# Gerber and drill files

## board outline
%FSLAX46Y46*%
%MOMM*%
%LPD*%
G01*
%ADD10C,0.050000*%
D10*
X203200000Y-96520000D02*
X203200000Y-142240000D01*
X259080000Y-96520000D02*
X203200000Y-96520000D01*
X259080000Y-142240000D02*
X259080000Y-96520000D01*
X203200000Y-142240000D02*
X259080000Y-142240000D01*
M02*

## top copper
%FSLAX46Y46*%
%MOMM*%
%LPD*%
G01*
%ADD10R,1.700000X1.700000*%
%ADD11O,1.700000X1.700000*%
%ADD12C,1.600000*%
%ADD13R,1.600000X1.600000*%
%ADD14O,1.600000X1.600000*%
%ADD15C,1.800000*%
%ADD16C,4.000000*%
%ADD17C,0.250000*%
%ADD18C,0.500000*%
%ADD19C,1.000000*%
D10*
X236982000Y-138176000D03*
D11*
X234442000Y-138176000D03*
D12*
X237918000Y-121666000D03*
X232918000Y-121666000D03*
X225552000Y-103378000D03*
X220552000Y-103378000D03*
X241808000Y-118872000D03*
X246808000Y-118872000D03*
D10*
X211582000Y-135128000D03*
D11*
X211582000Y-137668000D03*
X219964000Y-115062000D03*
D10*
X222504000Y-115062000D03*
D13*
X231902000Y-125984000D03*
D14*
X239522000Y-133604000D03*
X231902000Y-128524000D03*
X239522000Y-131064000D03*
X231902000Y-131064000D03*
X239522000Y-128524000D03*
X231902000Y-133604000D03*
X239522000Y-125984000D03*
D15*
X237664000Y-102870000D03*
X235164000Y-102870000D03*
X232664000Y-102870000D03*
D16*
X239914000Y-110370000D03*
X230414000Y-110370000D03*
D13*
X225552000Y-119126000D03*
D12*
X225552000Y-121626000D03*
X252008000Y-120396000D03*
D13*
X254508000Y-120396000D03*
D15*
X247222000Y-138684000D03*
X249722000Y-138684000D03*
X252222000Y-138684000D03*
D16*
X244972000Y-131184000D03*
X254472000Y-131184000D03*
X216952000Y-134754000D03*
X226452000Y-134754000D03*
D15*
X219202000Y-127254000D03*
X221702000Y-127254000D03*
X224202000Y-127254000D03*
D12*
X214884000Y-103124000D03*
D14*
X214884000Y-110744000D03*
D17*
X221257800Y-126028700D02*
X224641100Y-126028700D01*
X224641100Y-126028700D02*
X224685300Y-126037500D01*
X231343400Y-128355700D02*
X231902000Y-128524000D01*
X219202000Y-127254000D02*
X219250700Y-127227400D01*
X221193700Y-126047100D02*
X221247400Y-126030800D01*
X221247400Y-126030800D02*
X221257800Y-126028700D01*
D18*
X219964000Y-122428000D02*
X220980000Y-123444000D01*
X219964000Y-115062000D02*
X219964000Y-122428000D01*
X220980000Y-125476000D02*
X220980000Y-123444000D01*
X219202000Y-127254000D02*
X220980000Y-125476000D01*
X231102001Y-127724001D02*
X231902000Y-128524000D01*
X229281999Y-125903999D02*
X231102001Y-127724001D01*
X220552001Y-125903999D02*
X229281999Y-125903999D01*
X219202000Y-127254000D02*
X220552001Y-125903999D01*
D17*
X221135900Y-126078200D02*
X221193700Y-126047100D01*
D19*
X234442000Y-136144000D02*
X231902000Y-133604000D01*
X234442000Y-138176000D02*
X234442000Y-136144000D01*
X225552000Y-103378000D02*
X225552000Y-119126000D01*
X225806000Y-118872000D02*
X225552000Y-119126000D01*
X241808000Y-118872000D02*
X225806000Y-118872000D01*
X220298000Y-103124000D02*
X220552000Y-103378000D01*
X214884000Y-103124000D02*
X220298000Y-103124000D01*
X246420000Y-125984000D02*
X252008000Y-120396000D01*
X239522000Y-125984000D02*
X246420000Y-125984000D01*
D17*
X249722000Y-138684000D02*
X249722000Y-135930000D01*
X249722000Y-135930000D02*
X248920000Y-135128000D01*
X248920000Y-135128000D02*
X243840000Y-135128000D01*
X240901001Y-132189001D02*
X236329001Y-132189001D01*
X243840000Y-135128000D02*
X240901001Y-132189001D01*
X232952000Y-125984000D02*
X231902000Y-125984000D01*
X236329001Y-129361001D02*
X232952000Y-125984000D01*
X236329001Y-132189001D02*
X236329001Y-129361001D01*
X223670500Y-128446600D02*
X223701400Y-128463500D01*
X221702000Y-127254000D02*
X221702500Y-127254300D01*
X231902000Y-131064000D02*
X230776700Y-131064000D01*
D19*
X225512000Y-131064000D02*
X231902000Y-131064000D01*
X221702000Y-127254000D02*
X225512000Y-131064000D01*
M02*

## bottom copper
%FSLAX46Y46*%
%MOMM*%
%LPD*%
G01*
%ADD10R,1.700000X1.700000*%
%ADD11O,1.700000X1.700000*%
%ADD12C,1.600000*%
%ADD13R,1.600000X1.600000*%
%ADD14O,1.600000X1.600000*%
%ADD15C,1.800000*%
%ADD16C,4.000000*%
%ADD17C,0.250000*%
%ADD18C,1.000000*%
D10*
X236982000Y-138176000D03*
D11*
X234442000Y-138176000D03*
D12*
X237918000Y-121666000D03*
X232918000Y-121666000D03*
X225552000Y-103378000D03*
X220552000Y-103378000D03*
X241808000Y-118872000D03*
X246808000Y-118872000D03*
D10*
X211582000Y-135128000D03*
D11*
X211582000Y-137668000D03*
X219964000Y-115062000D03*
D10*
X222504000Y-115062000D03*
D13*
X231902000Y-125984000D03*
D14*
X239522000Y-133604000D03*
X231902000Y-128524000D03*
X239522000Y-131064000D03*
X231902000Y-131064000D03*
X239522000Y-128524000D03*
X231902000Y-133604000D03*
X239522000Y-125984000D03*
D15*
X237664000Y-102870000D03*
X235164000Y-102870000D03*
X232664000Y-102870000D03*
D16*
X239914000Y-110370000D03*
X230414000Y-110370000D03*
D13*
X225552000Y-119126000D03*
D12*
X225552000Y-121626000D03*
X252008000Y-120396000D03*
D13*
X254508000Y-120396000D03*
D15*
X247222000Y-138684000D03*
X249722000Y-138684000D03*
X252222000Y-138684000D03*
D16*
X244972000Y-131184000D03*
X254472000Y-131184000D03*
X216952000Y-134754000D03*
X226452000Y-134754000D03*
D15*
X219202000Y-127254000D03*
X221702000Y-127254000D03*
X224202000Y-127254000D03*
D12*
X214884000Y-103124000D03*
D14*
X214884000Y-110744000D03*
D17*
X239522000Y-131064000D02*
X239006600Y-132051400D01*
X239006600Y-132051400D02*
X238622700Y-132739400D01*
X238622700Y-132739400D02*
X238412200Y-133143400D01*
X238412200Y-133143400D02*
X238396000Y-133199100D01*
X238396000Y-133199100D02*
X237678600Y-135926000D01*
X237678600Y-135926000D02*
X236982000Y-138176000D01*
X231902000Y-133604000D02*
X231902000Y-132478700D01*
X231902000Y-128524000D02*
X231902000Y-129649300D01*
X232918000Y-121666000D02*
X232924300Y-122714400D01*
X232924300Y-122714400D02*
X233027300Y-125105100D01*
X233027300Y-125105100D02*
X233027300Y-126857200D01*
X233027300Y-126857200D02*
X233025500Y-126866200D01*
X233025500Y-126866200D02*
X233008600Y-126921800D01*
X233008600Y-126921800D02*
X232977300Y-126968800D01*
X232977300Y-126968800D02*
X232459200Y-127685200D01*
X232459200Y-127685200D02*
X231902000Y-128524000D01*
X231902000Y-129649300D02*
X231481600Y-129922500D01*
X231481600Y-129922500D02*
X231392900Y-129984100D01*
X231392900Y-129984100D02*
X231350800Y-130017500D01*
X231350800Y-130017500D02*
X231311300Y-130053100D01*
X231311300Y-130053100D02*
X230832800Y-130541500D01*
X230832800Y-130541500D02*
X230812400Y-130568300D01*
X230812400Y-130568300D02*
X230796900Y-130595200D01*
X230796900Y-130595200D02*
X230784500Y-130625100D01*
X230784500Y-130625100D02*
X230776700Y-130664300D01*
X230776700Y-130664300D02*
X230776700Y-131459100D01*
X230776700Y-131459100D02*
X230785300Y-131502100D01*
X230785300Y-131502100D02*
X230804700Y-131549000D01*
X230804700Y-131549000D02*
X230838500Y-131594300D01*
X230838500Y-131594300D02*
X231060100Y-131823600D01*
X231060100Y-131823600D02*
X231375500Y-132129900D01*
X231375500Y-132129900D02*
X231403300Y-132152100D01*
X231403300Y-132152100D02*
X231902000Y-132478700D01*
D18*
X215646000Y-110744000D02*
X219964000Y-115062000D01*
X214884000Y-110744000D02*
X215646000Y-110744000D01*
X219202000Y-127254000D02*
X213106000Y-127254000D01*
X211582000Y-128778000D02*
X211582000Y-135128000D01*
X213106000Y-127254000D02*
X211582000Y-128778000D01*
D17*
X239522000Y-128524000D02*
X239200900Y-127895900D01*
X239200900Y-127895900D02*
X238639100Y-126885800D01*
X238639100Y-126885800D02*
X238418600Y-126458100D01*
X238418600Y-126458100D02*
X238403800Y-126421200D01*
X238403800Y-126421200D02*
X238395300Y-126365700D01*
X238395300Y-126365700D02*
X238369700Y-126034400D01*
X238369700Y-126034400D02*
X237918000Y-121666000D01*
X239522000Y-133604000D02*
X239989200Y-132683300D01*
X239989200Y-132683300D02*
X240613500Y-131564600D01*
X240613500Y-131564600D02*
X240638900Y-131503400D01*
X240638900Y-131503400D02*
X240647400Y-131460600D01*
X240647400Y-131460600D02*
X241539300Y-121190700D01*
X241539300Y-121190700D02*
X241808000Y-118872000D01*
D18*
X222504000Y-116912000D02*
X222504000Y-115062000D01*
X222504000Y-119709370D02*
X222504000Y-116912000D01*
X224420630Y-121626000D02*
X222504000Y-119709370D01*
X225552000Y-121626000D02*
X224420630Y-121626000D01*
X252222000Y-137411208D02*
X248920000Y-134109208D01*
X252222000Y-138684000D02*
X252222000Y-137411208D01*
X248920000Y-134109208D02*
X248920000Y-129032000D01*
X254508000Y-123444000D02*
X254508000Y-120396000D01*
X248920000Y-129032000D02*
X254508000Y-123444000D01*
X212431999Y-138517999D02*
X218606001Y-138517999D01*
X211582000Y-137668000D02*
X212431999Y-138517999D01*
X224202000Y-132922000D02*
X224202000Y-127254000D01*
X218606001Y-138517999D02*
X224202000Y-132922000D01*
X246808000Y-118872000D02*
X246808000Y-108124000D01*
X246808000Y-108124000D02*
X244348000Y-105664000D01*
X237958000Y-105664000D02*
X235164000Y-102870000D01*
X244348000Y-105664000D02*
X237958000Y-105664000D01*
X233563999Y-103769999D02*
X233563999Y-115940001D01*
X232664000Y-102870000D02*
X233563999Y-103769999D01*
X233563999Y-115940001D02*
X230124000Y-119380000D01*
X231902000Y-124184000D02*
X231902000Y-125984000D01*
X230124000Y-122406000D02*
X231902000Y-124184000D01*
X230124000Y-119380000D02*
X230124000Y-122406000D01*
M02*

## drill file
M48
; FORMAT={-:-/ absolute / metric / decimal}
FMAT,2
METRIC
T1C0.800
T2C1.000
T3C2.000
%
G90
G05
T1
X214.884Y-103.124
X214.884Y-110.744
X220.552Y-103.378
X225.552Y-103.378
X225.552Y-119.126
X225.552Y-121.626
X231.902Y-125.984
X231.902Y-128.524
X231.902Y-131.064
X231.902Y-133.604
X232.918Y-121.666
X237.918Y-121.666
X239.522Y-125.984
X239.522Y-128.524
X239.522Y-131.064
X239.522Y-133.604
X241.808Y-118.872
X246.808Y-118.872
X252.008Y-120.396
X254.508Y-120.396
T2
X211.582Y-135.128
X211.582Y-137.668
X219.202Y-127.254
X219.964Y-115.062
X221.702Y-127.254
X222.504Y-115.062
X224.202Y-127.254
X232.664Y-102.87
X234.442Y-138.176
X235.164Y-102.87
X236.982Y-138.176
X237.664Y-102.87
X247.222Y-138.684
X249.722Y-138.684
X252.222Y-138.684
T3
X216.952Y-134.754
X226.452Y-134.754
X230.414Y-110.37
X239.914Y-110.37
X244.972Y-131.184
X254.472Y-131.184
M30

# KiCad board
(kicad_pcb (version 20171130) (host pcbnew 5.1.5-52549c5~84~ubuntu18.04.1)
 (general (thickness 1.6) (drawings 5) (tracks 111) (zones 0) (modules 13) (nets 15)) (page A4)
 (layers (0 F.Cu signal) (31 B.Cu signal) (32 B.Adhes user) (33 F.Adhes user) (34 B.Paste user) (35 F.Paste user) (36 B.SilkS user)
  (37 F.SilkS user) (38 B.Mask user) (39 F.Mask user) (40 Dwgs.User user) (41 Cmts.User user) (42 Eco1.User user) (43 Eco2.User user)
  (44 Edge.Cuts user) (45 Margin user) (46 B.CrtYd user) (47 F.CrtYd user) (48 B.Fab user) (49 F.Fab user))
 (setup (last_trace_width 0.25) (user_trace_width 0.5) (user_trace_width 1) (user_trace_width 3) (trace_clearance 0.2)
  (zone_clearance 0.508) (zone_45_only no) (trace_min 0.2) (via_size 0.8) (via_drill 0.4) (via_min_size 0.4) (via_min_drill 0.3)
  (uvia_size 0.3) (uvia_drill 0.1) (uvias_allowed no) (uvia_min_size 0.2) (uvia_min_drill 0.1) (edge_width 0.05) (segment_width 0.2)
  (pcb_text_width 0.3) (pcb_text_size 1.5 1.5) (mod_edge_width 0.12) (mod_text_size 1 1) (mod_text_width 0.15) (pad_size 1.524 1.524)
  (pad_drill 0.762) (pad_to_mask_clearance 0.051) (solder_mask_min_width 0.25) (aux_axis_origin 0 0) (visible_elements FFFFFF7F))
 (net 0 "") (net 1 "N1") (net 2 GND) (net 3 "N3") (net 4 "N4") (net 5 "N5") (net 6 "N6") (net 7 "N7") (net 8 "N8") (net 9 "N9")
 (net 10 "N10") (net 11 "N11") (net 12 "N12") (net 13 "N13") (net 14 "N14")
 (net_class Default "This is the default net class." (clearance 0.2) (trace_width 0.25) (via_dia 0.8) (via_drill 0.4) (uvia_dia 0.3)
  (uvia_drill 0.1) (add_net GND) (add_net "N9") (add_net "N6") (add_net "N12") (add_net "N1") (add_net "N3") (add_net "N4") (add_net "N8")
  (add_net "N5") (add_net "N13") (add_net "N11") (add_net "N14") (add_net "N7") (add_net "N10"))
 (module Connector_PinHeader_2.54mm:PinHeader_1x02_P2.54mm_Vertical (layer F.Cu) (at 236.982 138.176 270)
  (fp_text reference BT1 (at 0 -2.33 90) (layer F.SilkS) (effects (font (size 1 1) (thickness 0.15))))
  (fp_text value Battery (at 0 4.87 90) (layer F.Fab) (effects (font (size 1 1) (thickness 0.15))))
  (pad 1 thru_hole rect (at 0 0 270) (size 1.7 1.7) (drill 1) (layers *.Cu *.Mask) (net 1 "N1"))
  (pad 2 thru_hole oval (at 0 2.54 270) (size 1.7 1.7) (drill 1) (layers *.Cu *.Mask) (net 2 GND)))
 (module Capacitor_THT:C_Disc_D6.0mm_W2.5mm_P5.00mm (layer F.Cu) (at 232.918 121.666)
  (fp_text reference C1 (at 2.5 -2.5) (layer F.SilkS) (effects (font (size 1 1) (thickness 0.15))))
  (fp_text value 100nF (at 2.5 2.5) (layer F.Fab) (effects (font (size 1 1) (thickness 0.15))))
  (pad 2 thru_hole circle (at 5 0) (size 1.6 1.6) (drill 0.8) (layers *.Cu *.Mask) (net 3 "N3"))
  (pad 1 thru_hole circle (at 0 0) (size 1.6 1.6) (drill 0.8) (layers *.Cu *.Mask) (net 2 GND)))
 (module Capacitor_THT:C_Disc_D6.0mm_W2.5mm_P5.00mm (layer F.Cu) (at 225.552 103.378 180)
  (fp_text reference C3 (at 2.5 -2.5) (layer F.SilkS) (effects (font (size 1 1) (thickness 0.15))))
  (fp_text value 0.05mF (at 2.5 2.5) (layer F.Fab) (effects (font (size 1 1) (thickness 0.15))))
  (pad 1 thru_hole circle (at 0 0 180) (size 1.6 1.6) (drill 0.8) (layers *.Cu *.Mask) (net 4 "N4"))
  (pad 2 thru_hole circle (at 5 0 180) (size 1.6 1.6) (drill 0.8) (layers *.Cu *.Mask) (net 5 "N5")))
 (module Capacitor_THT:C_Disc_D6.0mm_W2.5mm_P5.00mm (layer F.Cu) (at 241.808 118.872)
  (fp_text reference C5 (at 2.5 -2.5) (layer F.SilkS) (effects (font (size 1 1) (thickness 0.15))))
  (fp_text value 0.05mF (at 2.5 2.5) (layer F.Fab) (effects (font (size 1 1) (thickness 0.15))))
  (pad 1 thru_hole circle (at 0 0) (size 1.6 1.6) (drill 0.8) (layers *.Cu *.Mask) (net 4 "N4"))
  (pad 2 thru_hole circle (at 5 0) (size 1.6 1.6) (drill 0.8) (layers *.Cu *.Mask) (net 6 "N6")))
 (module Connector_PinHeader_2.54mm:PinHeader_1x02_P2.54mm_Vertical (layer F.Cu) (at 211.582 135.128)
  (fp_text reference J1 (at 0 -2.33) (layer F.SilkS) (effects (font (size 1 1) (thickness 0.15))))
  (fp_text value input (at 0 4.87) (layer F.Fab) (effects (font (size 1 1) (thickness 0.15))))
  (pad 1 thru_hole rect (at 0 0) (size 1.7 1.7) (drill 1) (layers *.Cu *.Mask) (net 2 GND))
  (pad 2 thru_hole oval (at 0 2.54) (size 1.7 1.7) (drill 1) (layers *.Cu *.Mask) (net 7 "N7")))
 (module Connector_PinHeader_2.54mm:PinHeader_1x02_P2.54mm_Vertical (layer F.Cu) (at 222.504 115.062 270)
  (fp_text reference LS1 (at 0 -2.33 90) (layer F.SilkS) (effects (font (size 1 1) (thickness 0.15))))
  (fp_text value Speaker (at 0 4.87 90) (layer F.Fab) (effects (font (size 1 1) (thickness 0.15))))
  (pad 2 thru_hole oval (at 0 2.54 270) (size 1.7 1.7) (drill 1) (layers *.Cu *.Mask) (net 2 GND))
  (pad 1 thru_hole rect (at 0 0 270) (size 1.7 1.7) (drill 1) (layers *.Cu *.Mask) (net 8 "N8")))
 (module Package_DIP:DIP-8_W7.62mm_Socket (layer F.Cu) (at 231.902 125.984)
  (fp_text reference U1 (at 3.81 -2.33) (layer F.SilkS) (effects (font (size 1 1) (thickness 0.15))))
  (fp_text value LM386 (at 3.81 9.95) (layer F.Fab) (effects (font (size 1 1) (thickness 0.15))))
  (pad 1 thru_hole rect (at 0 0) (size 1.6 1.6) (drill 0.8) (layers *.Cu *.Mask) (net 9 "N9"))
  (pad 5 thru_hole oval (at 7.62 7.62) (size 1.6 1.6) (drill 0.8) (layers *.Cu *.Mask) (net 4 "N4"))
  (pad 2 thru_hole oval (at 0 2.54) (size 1.6 1.6) (drill 0.8) (layers *.Cu *.Mask) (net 2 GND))
  (pad 6 thru_hole oval (at 7.62 5.08) (size 1.6 1.6) (drill 0.8) (layers *.Cu *.Mask) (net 1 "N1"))
  (pad 3 thru_hole oval (at 0 5.08) (size 1.6 1.6) (drill 0.8) (layers *.Cu *.Mask) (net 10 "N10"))
  (pad 7 thru_hole oval (at 7.62 2.54) (size 1.6 1.6) (drill 0.8) (layers *.Cu *.Mask) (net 3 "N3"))
  (pad 4 thru_hole oval (at 0 7.62) (size 1.6 1.6) (drill 0.8) (layers *.Cu *.Mask) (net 2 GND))
  (pad 8 thru_hole oval (at 7.62 0) (size 1.6 1.6) (drill 0.8) (layers *.Cu *.Mask) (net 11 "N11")))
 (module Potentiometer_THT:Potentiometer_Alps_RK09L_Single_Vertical (layer F.Cu) (at 232.664 102.87 270)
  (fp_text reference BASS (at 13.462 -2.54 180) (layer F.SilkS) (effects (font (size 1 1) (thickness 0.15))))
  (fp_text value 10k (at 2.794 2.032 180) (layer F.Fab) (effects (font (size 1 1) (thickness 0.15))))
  (pad 3 thru_hole circle (at 0 -5 270) (size 1.8 1.8) (drill 1) (layers *.Cu *.Mask) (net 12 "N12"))
  (pad 2 thru_hole circle (at 0 -2.5 270) (size 1.8 1.8) (drill 1) (layers *.Cu *.Mask) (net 6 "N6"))
  (pad 1 thru_hole circle (at 0 0 270) (size 1.8 1.8) (drill 1) (layers *.Cu *.Mask) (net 9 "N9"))
  (pad "" np_thru_hole circle (at 7.5 -7.25 270) (size 4 4) (drill 2) (layers *.Cu *.Mask))
  (pad "" np_thru_hole circle (at 7.5 2.25 270) (size 4 4) (drill 2) (layers *.Cu *.Mask)))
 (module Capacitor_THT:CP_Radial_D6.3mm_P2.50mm (layer F.Cu) (at 225.552 119.126 270)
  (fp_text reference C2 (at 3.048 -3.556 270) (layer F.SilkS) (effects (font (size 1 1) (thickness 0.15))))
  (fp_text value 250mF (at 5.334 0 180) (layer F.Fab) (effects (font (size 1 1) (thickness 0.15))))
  (pad 1 thru_hole rect (at 0 0 270) (size 1.6 1.6) (drill 0.8) (layers *.Cu *.Mask) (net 4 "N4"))
  (pad 2 thru_hole circle (at 2.5 0 270) (size 1.6 1.6) (drill 0.8) (layers *.Cu *.Mask) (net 8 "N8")))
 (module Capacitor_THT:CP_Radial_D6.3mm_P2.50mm (layer F.Cu) (at 254.508 120.396 180)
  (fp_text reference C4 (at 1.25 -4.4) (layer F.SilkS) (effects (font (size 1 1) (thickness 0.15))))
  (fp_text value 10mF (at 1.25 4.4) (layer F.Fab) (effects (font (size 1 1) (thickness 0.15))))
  (pad 2 thru_hole circle (at 2.5 0 180) (size 1.6 1.6) (drill 0.8) (layers *.Cu *.Mask) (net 11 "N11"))
  (pad 1 thru_hole rect (at 0 0 180) (size 1.6 1.6) (drill 0.8) (layers *.Cu *.Mask) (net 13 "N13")))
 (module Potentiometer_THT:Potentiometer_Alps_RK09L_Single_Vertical (layer F.Cu) (at 252.222 138.684 90)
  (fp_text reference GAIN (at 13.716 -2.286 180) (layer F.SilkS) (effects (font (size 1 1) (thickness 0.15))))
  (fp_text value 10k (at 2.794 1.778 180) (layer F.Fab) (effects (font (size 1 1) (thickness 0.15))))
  (pad 3 thru_hole circle (at 0 -5 90) (size 1.8 1.8) (drill 1) (layers *.Cu *.Mask) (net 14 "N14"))
  (pad 2 thru_hole circle (at 0 -2.5 90) (size 1.8 1.8) (drill 1) (layers *.Cu *.Mask) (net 9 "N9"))
  (pad 1 thru_hole circle (at 0 0 90) (size 1.8 1.8) (drill 1) (layers *.Cu *.Mask) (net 13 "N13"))
  (pad "" np_thru_hole circle (at 7.5 -7.25 90) (size 4 4) (drill 2) (layers *.Cu *.Mask))
  (pad "" np_thru_hole circle (at 7.5 2.25 90) (size 4 4) (drill 2) (layers *.Cu *.Mask)))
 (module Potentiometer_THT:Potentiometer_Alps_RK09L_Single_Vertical (layer F.Cu) (at 219.202 127.254 270)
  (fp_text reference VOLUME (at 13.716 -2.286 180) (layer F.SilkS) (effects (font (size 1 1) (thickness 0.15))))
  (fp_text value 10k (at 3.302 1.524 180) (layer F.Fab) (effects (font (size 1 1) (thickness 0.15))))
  (pad "" np_thru_hole circle (at 7.5 2.25 270) (size 4 4) (drill 2) (layers *.Cu *.Mask))
  (pad "" np_thru_hole circle (at 7.5 -7.25 270) (size 4 4) (drill 2) (layers *.Cu *.Mask))
  (pad 1 thru_hole circle (at 0 0 270) (size 1.8 1.8) (drill 1) (layers *.Cu *.Mask) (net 2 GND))
  (pad 2 thru_hole circle (at 0 -2.5 270) (size 1.8 1.8) (drill 1) (layers *.Cu *.Mask) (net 10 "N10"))
  (pad 3 thru_hole circle (at 0 -5 270) (size 1.8 1.8) (drill 1) (layers *.Cu *.Mask) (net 7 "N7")))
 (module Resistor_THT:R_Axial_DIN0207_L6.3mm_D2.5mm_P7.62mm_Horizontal (layer F.Cu) (at 214.884 103.124 270)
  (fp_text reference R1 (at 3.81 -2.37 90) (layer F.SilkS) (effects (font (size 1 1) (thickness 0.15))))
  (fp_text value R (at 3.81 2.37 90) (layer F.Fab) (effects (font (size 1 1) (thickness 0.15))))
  (pad 1 thru_hole circle (at 0 0 270) (size 1.6 1.6) (drill 0.8) (layers *.Cu *.Mask) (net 5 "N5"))
  (pad 2 thru_hole oval (at 7.62 0 270) (size 1.6 1.6) (drill 0.8) (layers *.Cu *.Mask) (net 2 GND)))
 (gr_line (start 203.2 96.52) (end 203.2 142.24) (layer Edge.Cuts) (width 0.05))
 (gr_line (start 259.08 96.52) (end 203.2 96.52) (layer Edge.Cuts) (width 0.05))
 (gr_line (start 259.08 142.24) (end 259.08 96.52) (layer Edge.Cuts) (width 0.05))
 (gr_line (start 203.2 142.24) (end 259.08 142.24) (layer Edge.Cuts) (width 0.05))
 (segment (start 239.522 131.064) (end 239.0066 132.0514) (width 0.25) (layer B.Cu) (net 1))
 (segment (start 239.0066 132.0514) (end 238.6227 132.7394) (width 0.25) (layer B.Cu) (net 1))
 (segment (start 238.6227 132.7394) (end 238.4122 133.1434) (width 0.25) (layer B.Cu) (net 1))
 (segment (start 238.4122 133.1434) (end 238.396 133.1991) (width 0.25) (layer B.Cu) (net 1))
 (segment (start 238.396 133.1991) (end 237.6786 135.926) (width 0.25) (layer B.Cu) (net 1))
 (segment (start 237.6786 135.926) (end 236.982 138.176) (width 0.25) (layer B.Cu) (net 1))
 (segment (start 221.2578 126.0287) (end 224.6411 126.0287) (width 0.25) (layer F.Cu) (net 2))
 (segment (start 224.6411 126.0287) (end 224.6853 126.0375) (width 0.25) (layer F.Cu) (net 2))
 (segment (start 231.3434 128.3557) (end 231.902 128.524) (width 0.25) (layer F.Cu) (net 2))
 (segment (start 219.202 127.254) (end 219.2507 127.2274) (width 0.25) (layer F.Cu) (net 2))
 (segment (start 221.1937 126.0471) (end 221.2474 126.0308) (width 0.25) (layer F.Cu) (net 2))
 (segment (start 221.2474 126.0308) (end 221.2578 126.0287) (width 0.25) (layer F.Cu) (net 2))
 (segment (start 231.902 133.604) (end 231.902 132.4787) (width 0.25) (layer B.Cu) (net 2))
 (segment (start 231.902 128.524) (end 231.902 129.6493) (width 0.25) (layer B.Cu) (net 2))
 (segment (start 232.918 121.666) (end 232.9243 122.7144) (width 0.25) (layer B.Cu) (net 2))
 (segment (start 232.9243 122.7144) (end 233.0273 125.1051) (width 0.25) (layer B.Cu) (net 2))
 (segment (start 233.0273 125.1051) (end 233.0273 126.8572) (width 0.25) (layer B.Cu) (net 2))
 (segment (start 233.0273 126.8572) (end 233.0255 126.8662) (width 0.25) (layer B.Cu) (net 2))
 (segment (start 233.0255 126.8662) (end 233.0086 126.9218) (width 0.25) (layer B.Cu) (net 2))
 (segment (start 233.0086 126.9218) (end 232.9773 126.9688) (width 0.25) (layer B.Cu) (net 2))
 (segment (start 232.9773 126.9688) (end 232.4592 127.6852) (width 0.25) (layer B.Cu) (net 2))
 (segment (start 232.4592 127.6852) (end 231.902 128.524) (width 0.25) (layer B.Cu) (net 2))
 (segment (start 231.902 129.6493) (end 231.4816 129.9225) (width 0.25) (layer B.Cu) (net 2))
 (segment (start 231.4816 129.9225) (end 231.3929 129.9841) (width 0.25) (layer B.Cu) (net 2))
 (segment (start 231.3929 129.9841) (end 231.3508 130.0175) (width 0.25) (layer B.Cu) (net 2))
 (segment (start 231.3508 130.0175) (end 231.3113 130.0531) (width 0.25) (layer B.Cu) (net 2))
 (segment (start 231.3113 130.0531) (end 230.8328 130.5415) (width 0.25) (layer B.Cu) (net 2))
 (segment (start 230.8328 130.5415) (end 230.8124 130.5683) (width 0.25) (layer B.Cu) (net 2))
 (segment (start 230.8124 130.5683) (end 230.7969 130.5952) (width 0.25) (layer B.Cu) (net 2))
 (segment (start 230.7969 130.5952) (end 230.7845 130.6251) (width 0.25) (layer B.Cu) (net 2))
 (segment (start 230.7845 130.6251) (end 230.7767 130.6643) (width 0.25) (layer B.Cu) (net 2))
 (segment (start 230.7767 130.6643) (end 230.7767 131.4591) (width 0.25) (layer B.Cu) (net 2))
 (segment (start 230.7767 131.4591) (end 230.7853 131.5021) (width 0.25) (layer B.Cu) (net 2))
 (segment (start 230.7853 131.5021) (end 230.8047 131.549) (width 0.25) (layer B.Cu) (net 2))
 (segment (start 230.8047 131.549) (end 230.8385 131.5943) (width 0.25) (layer B.Cu) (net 2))
 (segment (start 230.8385 131.5943) (end 231.0601 131.8236) (width 0.25) (layer B.Cu) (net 2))
 (segment (start 231.0601 131.8236) (end 231.3755 132.1299) (width 0.25) (layer B.Cu) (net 2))
 (segment (start 231.3755 132.1299) (end 231.4033 132.1521) (width 0.25) (layer B.Cu) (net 2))
 (segment (start 231.4033 132.1521) (end 231.902 132.4787) (width 0.25) (layer B.Cu) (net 2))
 (segment (start 219.964 122.428) (end 220.98 123.444) (width 0.5) (layer F.Cu) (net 2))
 (segment (start 219.964 115.062) (end 219.964 122.428) (width 0.5) (layer F.Cu) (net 2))
 (segment (start 220.98 125.476) (end 220.98 123.444) (width 0.5) (layer F.Cu) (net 2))
 (segment (start 219.202 127.254) (end 220.98 125.476) (width 0.5) (layer F.Cu) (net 2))
 (segment (start 231.102001 127.724001) (end 231.902 128.524) (width 0.5) (layer F.Cu) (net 2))
 (segment (start 229.281999 125.903999) (end 231.102001 127.724001) (width 0.5) (layer F.Cu) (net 2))
 (segment (start 220.552001 125.903999) (end 229.281999 125.903999) (width 0.5) (layer F.Cu) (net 2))
 (segment (start 219.202 127.254) (end 220.552001 125.903999) (width 0.5) (layer F.Cu) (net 2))
 (segment (start 221.1359 126.0782) (end 221.1937 126.0471) (width 0.25) (layer F.Cu) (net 2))
 (segment (start 234.442 136.144) (end 231.902 133.604) (width 1) (layer F.Cu) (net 2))
 (segment (start 234.442 138.176) (end 234.442 136.144) (width 1) (layer F.Cu) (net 2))
 (segment (start 215.646 110.744) (end 219.964 115.062) (width 1) (layer B.Cu) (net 2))
 (segment (start 214.884 110.744) (end 215.646 110.744) (width 1) (layer B.Cu) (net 2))
 (segment (start 219.202 127.254) (end 213.106 127.254) (width 1) (layer B.Cu) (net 2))
 (segment (start 211.582 128.778) (end 211.582 135.128) (width 1) (layer B.Cu) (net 2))
 (segment (start 213.106 127.254) (end 211.582 128.778) (width 1) (layer B.Cu) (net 2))
 (segment (start 239.522 128.524) (end 239.2009 127.8959) (width 0.25) (layer B.Cu) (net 3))
 (segment (start 239.2009 127.8959) (end 238.6391 126.8858) (width 0.25) (layer B.Cu) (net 3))
 (segment (start 238.6391 126.8858) (end 238.4186 126.4581) (width 0.25) (layer B.Cu) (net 3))
 (segment (start 238.4186 126.4581) (end 238.4038 126.4212) (width 0.25) (layer B.Cu) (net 3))
 (segment (start 238.4038 126.4212) (end 238.3953 126.3657) (width 0.25) (layer B.Cu) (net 3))
 (segment (start 238.3953 126.3657) (end 238.3697 126.0344) (width 0.25) (layer B.Cu) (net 3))
 (segment (start 238.3697 126.0344) (end 237.918 121.666) (width 0.25) (layer B.Cu) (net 3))
 (segment (start 239.522 133.604) (end 239.9892 132.6833) (width 0.25) (layer B.Cu) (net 4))
 (segment (start 239.9892 132.6833) (end 240.6135 131.5646) (width 0.25) (layer B.Cu) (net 4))
 (segment (start 240.6135 131.5646) (end 240.6389 131.5034) (width 0.25) (layer B.Cu) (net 4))
 (segment (start 240.6389 131.5034) (end 240.6474 131.4606) (width 0.25) (layer B.Cu) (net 4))
 (segment (start 240.6474 131.4606) (end 241.5393 121.1907) (width 0.25) (layer B.Cu) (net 4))
 (segment (start 241.5393 121.1907) (end 241.808 118.872) (width 0.25) (layer B.Cu) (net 4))
 (segment (start 225.552 103.378) (end 225.552 119.126) (width 1) (layer F.Cu) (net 4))
 (segment (start 225.806 118.872) (end 225.552 119.126) (width 1) (layer F.Cu) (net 4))
 (segment (start 241.808 118.872) (end 225.806 118.872) (width 1) (layer F.Cu) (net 4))
 (segment (start 222.504 116.912) (end 222.504 115.062) (width 1) (layer B.Cu) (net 8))
 (segment (start 222.504 119.70937) (end 222.504 116.912) (width 1) (layer B.Cu) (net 8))
 (segment (start 224.42063 121.626) (end 222.504 119.70937) (width 1) (layer B.Cu) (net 8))
 (segment (start 225.552 121.626) (end 224.42063 121.626) (width 1) (layer B.Cu) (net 8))
 (segment (start 220.298 103.124) (end 220.552 103.378) (width 1) (layer F.Cu) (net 5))
 (segment (start 214.884 103.124) (end 220.298 103.124) (width 1) (layer F.Cu) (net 5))
 (segment (start 246.42 125.984) (end 252.008 120.396) (width 1) (layer F.Cu) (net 11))
 (segment (start 239.522 125.984) (end 246.42 125.984) (width 1) (layer F.Cu) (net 11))
 (segment (start 252.222 137.411208) (end 248.92 134.109208) (width 1) (layer B.Cu) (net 13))
 (segment (start 252.222 138.684) (end 252.222 137.411208) (width 1) (layer B.Cu) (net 13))
 (segment (start 248.92 134.109208) (end 248.92 129.032) (width 1) (layer B.Cu) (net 13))
 (segment (start 254.508 123.444) (end 254.508 120.396) (width 1) (layer B.Cu) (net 13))
 (segment (start 248.92 129.032) (end 254.508 123.444) (width 1) (layer B.Cu) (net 13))
 (segment (start 212.431999 138.517999) (end 218.606001 138.517999) (width 1) (layer B.Cu) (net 7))
 (segment (start 211.582 137.668) (end 212.431999 138.517999) (width 1) (layer B.Cu) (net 7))
 (segment (start 224.202 132.922) (end 224.202 127.254) (width 1) (layer B.Cu) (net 7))
 (segment (start 218.606001 138.517999) (end 224.202 132.922) (width 1) (layer B.Cu) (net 7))
 (segment (start 246.808 118.872) (end 246.808 108.124) (width 1) (layer B.Cu) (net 6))
 (segment (start 246.808 108.124) (end 244.348 105.664) (width 1) (layer B.Cu) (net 6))
 (segment (start 237.958 105.664) (end 235.164 102.87) (width 1) (layer B.Cu) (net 6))
 (segment (start 244.348 105.664) (end 237.958 105.664) (width 1) (layer B.Cu) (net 6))
 (segment (start 249.722 138.684) (end 249.722 135.93) (width 0.25) (layer F.Cu) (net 9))
 (segment (start 249.722 135.93) (end 248.92 135.128) (width 0.25) (layer F.Cu) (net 9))
 (segment (start 248.92 135.128) (end 243.84 135.128) (width 0.25) (layer F.Cu) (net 9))
 (segment (start 240.901001 132.189001) (end 236.329001 132.189001) (width 0.25) (layer F.Cu) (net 9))
 (segment (start 243.84 135.128) (end 240.901001 132.189001) (width 0.25) (layer F.Cu) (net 9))
 (segment (start 232.952 125.984) (end 231.902 125.984) (width 0.25) (layer F.Cu) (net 9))
 (segment (start 236.329001 129.361001) (end 232.952 125.984) (width 0.25) (layer F.Cu) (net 9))
 (segment (start 236.329001 132.189001) (end 236.329001 129.361001) (width 0.25) (layer F.Cu) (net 9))
 (segment (start 233.563999 103.769999) (end 233.563999 115.940001) (width 1) (layer B.Cu) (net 9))
 (segment (start 232.664 102.87) (end 233.563999 103.769999) (width 1) (layer B.Cu) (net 9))
 (segment (start 233.563999 115.940001) (end 230.124 119.38) (width 1) (layer B.Cu) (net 9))
 (segment (start 231.902 124.184) (end 231.902 125.984) (width 1) (layer B.Cu) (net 9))
 (segment (start 230.124 122.406) (end 231.902 124.184) (width 1) (layer B.Cu) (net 9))
 (segment (start 230.124 119.38) (end 230.124 122.406) (width 1) (layer B.Cu) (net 9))
 (segment (start 223.6705 128.4466) (end 223.7014 128.4635) (width 0.25) (layer F.Cu) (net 10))
 (segment (start 221.702 127.254) (end 221.7025 127.2543) (width 0.25) (layer F.Cu) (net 10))
 (segment (start 231.902 131.064) (end 230.7767 131.064) (width 0.25) (layer F.Cu) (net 10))
 (segment (start 225.512 131.064) (end 231.902 131.064) (width 1) (layer F.Cu) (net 10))
 (segment (start 221.702 127.254) (end 225.512 131.064) (width 1) (layer F.Cu) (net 10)))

